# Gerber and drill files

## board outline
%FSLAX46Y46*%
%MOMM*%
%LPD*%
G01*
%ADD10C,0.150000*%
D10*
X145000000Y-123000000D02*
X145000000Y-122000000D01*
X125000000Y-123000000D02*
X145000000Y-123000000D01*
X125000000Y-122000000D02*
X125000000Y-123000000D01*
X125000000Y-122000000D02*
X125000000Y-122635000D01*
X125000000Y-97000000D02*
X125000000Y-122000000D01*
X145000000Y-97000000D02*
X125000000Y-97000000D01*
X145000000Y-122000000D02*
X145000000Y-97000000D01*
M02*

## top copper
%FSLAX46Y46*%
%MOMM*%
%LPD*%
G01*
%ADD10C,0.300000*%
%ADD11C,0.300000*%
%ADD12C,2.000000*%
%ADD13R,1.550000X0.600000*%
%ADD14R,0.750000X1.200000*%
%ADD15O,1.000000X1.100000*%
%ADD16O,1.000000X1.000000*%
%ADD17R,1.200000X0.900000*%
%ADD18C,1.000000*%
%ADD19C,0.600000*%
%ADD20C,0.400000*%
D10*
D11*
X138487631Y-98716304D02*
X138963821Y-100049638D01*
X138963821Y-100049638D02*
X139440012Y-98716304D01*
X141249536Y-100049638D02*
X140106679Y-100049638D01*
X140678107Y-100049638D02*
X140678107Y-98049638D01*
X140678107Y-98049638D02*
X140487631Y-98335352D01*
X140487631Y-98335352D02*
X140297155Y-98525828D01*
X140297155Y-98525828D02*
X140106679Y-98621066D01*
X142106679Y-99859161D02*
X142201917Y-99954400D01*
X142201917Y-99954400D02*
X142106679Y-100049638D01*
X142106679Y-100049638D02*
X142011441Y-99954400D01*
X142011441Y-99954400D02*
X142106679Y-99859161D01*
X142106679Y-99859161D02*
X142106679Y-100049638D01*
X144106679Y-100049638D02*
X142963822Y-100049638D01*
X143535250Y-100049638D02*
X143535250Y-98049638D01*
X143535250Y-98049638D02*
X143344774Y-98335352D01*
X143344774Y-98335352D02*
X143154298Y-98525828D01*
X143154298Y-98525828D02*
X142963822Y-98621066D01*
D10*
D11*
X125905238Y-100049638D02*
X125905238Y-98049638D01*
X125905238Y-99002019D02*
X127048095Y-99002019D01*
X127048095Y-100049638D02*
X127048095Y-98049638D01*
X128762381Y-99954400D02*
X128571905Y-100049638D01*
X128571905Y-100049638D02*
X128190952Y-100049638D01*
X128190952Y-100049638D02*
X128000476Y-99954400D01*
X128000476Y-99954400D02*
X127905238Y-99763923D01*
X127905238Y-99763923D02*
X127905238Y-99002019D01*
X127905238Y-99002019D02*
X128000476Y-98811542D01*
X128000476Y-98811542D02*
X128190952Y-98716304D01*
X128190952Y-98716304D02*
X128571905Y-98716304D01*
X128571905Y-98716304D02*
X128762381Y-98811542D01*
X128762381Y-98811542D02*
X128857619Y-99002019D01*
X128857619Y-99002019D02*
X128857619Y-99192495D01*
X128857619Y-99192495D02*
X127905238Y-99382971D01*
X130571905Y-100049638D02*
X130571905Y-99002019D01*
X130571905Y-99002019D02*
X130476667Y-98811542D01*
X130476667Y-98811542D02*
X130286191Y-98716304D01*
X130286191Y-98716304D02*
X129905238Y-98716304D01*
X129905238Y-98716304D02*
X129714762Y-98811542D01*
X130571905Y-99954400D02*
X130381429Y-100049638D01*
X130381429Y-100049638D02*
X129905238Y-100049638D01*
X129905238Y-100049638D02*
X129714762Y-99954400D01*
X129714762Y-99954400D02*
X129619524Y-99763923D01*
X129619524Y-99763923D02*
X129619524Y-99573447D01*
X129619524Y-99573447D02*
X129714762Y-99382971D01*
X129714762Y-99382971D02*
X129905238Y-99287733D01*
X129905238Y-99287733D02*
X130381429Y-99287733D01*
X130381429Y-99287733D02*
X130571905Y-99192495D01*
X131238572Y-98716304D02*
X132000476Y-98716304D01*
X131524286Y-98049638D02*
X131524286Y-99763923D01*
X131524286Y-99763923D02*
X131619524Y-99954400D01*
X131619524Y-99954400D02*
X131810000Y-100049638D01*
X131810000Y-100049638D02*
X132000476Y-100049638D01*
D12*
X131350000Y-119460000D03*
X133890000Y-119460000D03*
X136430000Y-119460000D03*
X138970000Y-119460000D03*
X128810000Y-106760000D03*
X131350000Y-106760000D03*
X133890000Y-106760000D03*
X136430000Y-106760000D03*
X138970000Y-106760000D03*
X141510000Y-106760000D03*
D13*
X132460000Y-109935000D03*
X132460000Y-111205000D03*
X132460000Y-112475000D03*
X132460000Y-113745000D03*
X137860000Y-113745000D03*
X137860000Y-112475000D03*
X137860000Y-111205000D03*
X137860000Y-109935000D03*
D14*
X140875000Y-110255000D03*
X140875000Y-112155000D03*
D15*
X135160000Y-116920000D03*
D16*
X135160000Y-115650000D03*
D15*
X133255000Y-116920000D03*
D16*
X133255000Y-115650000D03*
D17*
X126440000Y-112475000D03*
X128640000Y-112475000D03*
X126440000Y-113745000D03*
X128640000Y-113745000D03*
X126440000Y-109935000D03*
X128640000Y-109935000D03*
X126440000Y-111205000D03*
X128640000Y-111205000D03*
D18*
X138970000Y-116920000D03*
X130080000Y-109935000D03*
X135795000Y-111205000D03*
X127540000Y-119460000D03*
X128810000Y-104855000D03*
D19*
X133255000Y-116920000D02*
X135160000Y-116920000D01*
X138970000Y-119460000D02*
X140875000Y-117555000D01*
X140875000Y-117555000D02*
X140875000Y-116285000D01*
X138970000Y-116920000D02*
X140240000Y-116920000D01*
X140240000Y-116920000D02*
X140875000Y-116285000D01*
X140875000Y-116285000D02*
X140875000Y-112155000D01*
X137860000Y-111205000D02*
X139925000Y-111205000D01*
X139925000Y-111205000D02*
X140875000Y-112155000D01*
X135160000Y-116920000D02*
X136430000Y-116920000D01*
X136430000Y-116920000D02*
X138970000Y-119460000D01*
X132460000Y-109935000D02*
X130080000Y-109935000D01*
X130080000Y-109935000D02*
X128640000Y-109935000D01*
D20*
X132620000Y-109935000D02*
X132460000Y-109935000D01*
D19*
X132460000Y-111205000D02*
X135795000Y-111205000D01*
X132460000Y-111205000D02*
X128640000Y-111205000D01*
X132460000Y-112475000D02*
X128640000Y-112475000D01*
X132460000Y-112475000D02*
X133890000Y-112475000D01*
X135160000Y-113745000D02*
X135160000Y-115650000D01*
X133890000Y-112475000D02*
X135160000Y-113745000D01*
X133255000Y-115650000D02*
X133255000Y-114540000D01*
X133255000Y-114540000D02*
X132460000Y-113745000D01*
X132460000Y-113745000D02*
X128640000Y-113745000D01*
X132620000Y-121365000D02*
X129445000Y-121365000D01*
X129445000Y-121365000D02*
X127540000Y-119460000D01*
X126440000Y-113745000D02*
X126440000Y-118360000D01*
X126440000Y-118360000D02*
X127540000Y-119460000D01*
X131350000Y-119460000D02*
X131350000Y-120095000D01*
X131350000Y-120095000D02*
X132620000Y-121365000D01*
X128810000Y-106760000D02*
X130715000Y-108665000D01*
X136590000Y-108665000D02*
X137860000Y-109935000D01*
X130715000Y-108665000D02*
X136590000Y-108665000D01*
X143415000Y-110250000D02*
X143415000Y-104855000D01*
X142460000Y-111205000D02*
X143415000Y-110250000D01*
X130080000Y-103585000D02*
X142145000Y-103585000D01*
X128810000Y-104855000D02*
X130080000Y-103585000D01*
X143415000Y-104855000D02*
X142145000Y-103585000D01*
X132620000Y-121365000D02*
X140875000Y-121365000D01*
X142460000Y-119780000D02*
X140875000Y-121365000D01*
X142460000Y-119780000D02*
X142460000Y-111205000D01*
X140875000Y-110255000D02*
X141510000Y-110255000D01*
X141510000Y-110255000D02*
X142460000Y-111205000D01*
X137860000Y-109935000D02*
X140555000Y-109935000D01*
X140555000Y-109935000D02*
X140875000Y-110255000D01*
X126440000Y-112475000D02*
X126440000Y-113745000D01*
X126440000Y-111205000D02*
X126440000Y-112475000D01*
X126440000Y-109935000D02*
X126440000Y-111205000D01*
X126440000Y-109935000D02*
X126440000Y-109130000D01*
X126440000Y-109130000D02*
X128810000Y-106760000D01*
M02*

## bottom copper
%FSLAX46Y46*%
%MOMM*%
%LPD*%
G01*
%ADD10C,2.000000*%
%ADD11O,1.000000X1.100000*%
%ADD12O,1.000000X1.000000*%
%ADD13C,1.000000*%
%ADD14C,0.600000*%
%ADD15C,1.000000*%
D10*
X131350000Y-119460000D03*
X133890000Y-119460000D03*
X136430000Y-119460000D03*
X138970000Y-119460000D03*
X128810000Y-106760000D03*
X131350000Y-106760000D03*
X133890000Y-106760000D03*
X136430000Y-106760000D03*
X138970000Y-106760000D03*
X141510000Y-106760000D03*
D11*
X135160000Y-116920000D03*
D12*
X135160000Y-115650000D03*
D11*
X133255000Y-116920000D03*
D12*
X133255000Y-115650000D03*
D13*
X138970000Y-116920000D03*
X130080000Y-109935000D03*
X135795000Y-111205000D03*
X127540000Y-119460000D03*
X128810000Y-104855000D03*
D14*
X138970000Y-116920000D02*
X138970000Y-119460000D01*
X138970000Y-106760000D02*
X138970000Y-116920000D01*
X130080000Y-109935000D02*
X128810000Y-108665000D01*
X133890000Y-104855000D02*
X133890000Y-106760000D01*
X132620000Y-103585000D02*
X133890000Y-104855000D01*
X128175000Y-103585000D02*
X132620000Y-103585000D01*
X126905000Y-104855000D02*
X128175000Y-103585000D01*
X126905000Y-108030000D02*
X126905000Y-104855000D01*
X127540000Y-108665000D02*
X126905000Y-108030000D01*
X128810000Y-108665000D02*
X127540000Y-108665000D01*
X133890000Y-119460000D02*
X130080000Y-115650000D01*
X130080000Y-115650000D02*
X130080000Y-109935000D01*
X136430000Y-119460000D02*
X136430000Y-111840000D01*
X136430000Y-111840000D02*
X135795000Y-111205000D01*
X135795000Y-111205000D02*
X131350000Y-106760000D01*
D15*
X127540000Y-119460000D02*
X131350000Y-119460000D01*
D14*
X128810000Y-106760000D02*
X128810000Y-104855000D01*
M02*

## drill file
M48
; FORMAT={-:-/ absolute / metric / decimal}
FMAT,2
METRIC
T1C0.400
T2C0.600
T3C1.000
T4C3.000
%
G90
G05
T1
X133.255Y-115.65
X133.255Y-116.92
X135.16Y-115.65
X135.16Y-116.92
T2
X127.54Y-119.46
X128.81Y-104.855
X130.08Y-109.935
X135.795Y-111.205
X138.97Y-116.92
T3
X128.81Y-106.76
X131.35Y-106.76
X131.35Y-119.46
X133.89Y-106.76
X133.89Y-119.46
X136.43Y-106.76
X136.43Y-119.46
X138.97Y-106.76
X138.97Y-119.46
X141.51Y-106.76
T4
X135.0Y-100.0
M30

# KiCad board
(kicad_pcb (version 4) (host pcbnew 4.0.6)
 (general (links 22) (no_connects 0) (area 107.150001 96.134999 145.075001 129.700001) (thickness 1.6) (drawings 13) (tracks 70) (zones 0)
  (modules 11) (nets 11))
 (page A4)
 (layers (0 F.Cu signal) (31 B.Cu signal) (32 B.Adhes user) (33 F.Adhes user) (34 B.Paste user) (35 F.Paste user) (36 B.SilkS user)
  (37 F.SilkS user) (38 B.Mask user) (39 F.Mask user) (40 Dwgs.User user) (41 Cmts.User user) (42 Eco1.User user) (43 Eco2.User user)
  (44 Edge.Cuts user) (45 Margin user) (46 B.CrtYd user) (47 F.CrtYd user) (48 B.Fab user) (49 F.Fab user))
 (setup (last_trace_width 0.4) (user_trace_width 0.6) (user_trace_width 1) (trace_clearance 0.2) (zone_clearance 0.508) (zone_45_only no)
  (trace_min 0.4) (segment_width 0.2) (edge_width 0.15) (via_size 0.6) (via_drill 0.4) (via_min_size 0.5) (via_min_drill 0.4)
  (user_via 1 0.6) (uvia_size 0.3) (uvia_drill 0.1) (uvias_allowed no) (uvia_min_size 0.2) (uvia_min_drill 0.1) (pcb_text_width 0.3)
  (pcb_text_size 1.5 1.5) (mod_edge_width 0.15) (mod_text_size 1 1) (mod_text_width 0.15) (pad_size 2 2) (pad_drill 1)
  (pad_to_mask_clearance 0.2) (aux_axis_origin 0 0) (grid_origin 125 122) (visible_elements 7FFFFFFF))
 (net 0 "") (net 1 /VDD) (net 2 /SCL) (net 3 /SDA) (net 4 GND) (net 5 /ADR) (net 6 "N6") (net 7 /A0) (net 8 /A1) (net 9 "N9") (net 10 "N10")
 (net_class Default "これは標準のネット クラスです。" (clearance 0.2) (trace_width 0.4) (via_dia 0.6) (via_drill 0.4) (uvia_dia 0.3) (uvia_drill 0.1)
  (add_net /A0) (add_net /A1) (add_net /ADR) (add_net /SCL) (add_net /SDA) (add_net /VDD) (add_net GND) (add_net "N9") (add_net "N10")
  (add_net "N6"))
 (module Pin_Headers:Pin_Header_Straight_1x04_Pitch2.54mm (layer F.Cu) (at 131.35 119.46 90)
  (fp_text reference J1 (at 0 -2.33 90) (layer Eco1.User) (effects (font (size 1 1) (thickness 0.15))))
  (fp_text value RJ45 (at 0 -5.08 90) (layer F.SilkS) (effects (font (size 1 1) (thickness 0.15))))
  (pad 1 thru_hole circle (at 0 0 90) (size 2 2) (drill 1) (layers *.Cu *.Mask) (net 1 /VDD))
  (pad 2 thru_hole circle (at 0 2.54 90) (size 2 2) (drill 1) (layers *.Cu *.Mask) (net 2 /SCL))
  (pad 3 thru_hole circle (at 0 5.08 90) (size 2 2) (drill 1) (layers *.Cu *.Mask) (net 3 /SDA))
  (pad 4 thru_hole circle (at 0 7.62 90) (size 2 2) (drill 1) (layers *.Cu *.Mask) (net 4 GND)))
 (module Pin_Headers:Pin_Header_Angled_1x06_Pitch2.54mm (layer F.Cu) (at 128.81 106.76 90)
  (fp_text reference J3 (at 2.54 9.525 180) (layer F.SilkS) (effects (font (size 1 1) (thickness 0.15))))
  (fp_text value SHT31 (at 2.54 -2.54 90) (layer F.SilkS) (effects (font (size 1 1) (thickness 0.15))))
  (pad 1 thru_hole circle (at 0 0 90) (size 2 2) (drill 1) (layers *.Cu *.Mask) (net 1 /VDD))
  (pad 2 thru_hole circle (at 0 2.54 90) (size 2 2) (drill 1) (layers *.Cu *.Mask) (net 3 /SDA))
  (pad 3 thru_hole circle (at 0 5.08 90) (size 2 2) (drill 1) (layers *.Cu *.Mask) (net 2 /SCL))
  (pad 4 thru_hole circle (at 0 7.62 90) (size 2 2) (drill 1) (layers *.Cu *.Mask) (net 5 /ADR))
  (pad 5 thru_hole circle (at 0 10.16 90) (size 2 2) (drill 1) (layers *.Cu *.Mask) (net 4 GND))
  (pad 6 thru_hole circle (at 0 12.7 90) (size 2 2) (drill 1) (layers *.Cu *.Mask) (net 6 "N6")))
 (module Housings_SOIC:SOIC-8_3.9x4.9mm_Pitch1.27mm (layer F.Cu) (at 135.16 111.84)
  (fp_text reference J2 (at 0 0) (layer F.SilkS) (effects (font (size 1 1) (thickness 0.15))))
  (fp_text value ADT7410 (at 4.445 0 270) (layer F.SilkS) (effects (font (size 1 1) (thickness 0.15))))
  (pad 1 smd rect (at -2.7 -1.905) (size 1.55 0.6) (layers F.Cu F.Paste F.Mask) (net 2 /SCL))
  (pad 2 smd rect (at -2.7 -0.635) (size 1.55 0.6) (layers F.Cu F.Paste F.Mask) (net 3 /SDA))
  (pad 3 smd rect (at -2.7 0.635) (size 1.55 0.6) (layers F.Cu F.Paste F.Mask) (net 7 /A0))
  (pad 4 smd rect (at -2.7 1.905) (size 1.55 0.6) (layers F.Cu F.Paste F.Mask) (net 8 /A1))
  (pad 5 smd rect (at 2.7 1.905) (size 1.55 0.6) (layers F.Cu F.Paste F.Mask) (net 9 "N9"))
  (pad 6 smd rect (at 2.7 0.635) (size 1.55 0.6) (layers F.Cu F.Paste F.Mask) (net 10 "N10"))
  (pad 7 smd rect (at 2.7 -0.635) (size 1.55 0.6) (layers F.Cu F.Paste F.Mask) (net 4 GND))
  (pad 8 smd rect (at 2.7 -1.905) (size 1.55 0.6) (layers F.Cu F.Paste F.Mask) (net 1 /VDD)))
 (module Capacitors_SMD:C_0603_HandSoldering (layer F.Cu) (at 140.875 111.205 270)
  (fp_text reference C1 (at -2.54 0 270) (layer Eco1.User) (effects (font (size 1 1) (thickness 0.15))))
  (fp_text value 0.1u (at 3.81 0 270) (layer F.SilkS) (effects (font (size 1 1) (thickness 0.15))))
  (pad 1 smd rect (at -0.95 0 270) (size 1.2 0.75) (layers F.Cu F.Paste F.Mask) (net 1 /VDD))
  (pad 2 smd rect (at 0.95 0 270) (size 1.2 0.75) (layers F.Cu F.Paste F.Mask) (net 4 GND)))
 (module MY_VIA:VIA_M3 (layer F.Cu) (at 135 100)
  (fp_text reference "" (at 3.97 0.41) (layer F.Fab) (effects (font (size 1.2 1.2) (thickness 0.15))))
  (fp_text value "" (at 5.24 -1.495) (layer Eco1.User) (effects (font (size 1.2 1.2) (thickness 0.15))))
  (pad "" np_thru_hole oval (at 0 0) (size 3 3) (drill 3) (layers *.Cu *.Mask)))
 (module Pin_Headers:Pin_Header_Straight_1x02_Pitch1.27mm (layer F.Cu) (at 135.16 116.92 180)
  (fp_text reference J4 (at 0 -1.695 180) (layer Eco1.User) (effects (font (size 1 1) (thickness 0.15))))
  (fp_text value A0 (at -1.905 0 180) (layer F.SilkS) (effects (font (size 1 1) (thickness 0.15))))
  (pad 1 thru_hole oval (at 0 0 180) (size 1 1.1) (drill 0.4) (layers *.Cu *.Mask) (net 4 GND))
  (pad 2 thru_hole oval (at 0 1.27 180) (size 1 1) (drill 0.4) (layers *.Cu *.Mask) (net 7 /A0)))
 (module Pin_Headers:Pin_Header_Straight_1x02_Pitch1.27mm (layer F.Cu) (at 133.255 116.92 180)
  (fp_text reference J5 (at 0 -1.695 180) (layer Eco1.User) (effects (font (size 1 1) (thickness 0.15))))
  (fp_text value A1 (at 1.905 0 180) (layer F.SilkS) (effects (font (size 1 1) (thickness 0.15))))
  (pad 1 thru_hole oval (at 0 0 180) (size 1 1.1) (drill 0.4) (layers *.Cu *.Mask) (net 4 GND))
  (pad 2 thru_hole oval (at 0 1.27 180) (size 1 1) (drill 0.4) (layers *.Cu *.Mask) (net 8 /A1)))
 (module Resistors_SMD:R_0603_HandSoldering (layer F.Cu) (at 127.54 112.475)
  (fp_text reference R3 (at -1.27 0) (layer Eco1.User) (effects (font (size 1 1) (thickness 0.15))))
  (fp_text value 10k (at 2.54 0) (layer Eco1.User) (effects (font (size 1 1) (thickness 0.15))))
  (pad 1 smd rect (at -1.1 0) (size 1.2 0.9) (layers F.Cu F.Paste F.Mask) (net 1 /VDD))
  (pad 2 smd rect (at 1.1 0) (size 1.2 0.9) (layers F.Cu F.Paste F.Mask) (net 7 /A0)))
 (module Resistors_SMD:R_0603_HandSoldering (layer F.Cu) (at 127.54 113.745)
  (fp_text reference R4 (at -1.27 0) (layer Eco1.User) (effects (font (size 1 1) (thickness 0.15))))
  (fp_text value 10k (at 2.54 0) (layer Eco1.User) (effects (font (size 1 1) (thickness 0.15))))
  (pad 1 smd rect (at -1.1 0) (size 1.2 0.9) (layers F.Cu F.Paste F.Mask) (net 1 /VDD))
  (pad 2 smd rect (at 1.1 0) (size 1.2 0.9) (layers F.Cu F.Paste F.Mask) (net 8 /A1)))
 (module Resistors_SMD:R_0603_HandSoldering (layer F.Cu) (at 127.54 109.935)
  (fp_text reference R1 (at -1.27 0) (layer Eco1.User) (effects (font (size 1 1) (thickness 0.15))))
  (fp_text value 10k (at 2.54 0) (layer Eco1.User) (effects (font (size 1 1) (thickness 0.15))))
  (pad 1 smd rect (at -1.1 0) (size 1.2 0.9) (layers F.Cu F.Paste F.Mask) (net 1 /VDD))
  (pad 2 smd rect (at 1.1 0) (size 1.2 0.9) (layers F.Cu F.Paste F.Mask) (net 2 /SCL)))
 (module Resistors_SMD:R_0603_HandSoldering (layer F.Cu) (at 127.54 111.205)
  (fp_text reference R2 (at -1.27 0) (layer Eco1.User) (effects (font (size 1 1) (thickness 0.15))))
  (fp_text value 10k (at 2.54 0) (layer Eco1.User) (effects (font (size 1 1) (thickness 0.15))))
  (pad 1 smd rect (at -1.1 0) (size 1.2 0.9) (layers F.Cu F.Paste F.Mask) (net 1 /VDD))
  (pad 2 smd rect (at 1.1 0) (size 1.2 0.9) (layers F.Cu F.Paste F.Mask) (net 3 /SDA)))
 (gr_line (start 145 123) (end 145 122) (angle 90) (layer Edge.Cuts) (width 0.15))
 (gr_line (start 125 123) (end 145 123) (angle 90) (layer Edge.Cuts) (width 0.15))
 (gr_line (start 125 122) (end 125 123) (angle 90) (layer Edge.Cuts) (width 0.15))
 (gr_line (start 125 122) (end 125 122.635) (angle 90) (layer Edge.Cuts) (width 0.15))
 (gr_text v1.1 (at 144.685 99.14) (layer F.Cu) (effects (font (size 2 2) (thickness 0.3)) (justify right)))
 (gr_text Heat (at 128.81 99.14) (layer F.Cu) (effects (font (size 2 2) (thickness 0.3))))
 (gr_line (start 125 97) (end 125 122) (angle 90) (layer Edge.Cuts) (width 0.15))
 (gr_line (start 145 97) (end 125 97) (angle 90) (layer Edge.Cuts) (width 0.15))
 (gr_line (start 145 122) (end 145 97) (angle 90) (layer Edge.Cuts) (width 0.15))
 (segment (start 133.255 116.92) (end 135.16 116.92) (width 0.6) (layer F.Cu) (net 4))
 (segment (start 138.97 116.92) (end 138.97 119.46) (width 0.6) (layer B.Cu) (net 4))
 (segment (start 138.97 119.46) (end 140.875 117.555) (width 0.6) (layer F.Cu) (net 4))
 (segment (start 140.875 117.555) (end 140.875 116.285) (width 0.6) (layer F.Cu) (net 4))
 (segment (start 138.97 116.92) (end 140.24 116.92) (width 0.6) (layer F.Cu) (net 4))
 (segment (start 140.24 116.92) (end 140.875 116.285) (width 0.6) (layer F.Cu) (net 4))
 (via (at 138.97 116.92) (size 1) (drill 0.6) (layers F.Cu B.Cu) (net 4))
 (segment (start 140.875 116.285) (end 140.875 112.155) (width 0.6) (layer F.Cu) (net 4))
 (segment (start 137.86 111.205) (end 139.925 111.205) (width 0.6) (layer F.Cu) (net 4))
 (segment (start 139.925 111.205) (end 140.875 112.155) (width 0.6) (layer F.Cu) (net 4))
 (segment (start 138.97 106.76) (end 138.97 116.92) (width 0.6) (layer B.Cu) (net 4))
 (segment (start 135.16 116.92) (end 136.43 116.92) (width 0.6) (layer F.Cu) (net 4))
 (segment (start 136.43 116.92) (end 138.97 119.46) (width 0.6) (layer F.Cu) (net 4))
 (segment (start 130.08 109.935) (end 128.81 108.665) (width 0.6) (layer B.Cu) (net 2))
 (segment (start 133.89 104.855) (end 133.89 106.76) (width 0.6) (layer B.Cu) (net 2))
 (segment (start 132.62 103.585) (end 133.89 104.855) (width 0.6) (layer B.Cu) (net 2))
 (segment (start 128.175 103.585) (end 132.62 103.585) (width 0.6) (layer B.Cu) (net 2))
 (segment (start 126.905 104.855) (end 128.175 103.585) (width 0.6) (layer B.Cu) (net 2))
 (segment (start 126.905 108.03) (end 126.905 104.855) (width 0.6) (layer B.Cu) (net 2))
 (segment (start 127.54 108.665) (end 126.905 108.03) (width 0.6) (layer B.Cu) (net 2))
 (segment (start 128.81 108.665) (end 127.54 108.665) (width 0.6) (layer B.Cu) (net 2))
 (segment (start 133.89 119.46) (end 130.08 115.65) (width 0.6) (layer B.Cu) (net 2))
 (via (at 130.08 109.935) (size 1) (drill 0.6) (layers F.Cu B.Cu) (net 2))
 (segment (start 130.08 115.65) (end 130.08 109.935) (width 0.6) (layer B.Cu) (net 2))
 (segment (start 132.46 109.935) (end 130.08 109.935) (width 0.6) (layer F.Cu) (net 2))
 (segment (start 130.08 109.935) (end 128.64 109.935) (width 0.6) (layer F.Cu) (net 2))
 (segment (start 132.62 109.935) (end 132.46 109.935) (width 0.4) (layer F.Cu) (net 2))
 (segment (start 132.46 111.205) (end 135.795 111.205) (width 0.6) (layer F.Cu) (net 3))
 (via (at 135.795 111.205) (size 1) (drill 0.6) (layers F.Cu B.Cu) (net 3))
 (segment (start 136.43 119.46) (end 136.43 111.84) (width 0.6) (layer B.Cu) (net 3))
 (segment (start 136.43 111.84) (end 135.795 111.205) (width 0.6) (layer B.Cu) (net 3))
 (segment (start 135.795 111.205) (end 131.35 106.76) (width 0.6) (layer B.Cu) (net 3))
 (segment (start 132.46 111.205) (end 128.64 111.205) (width 0.6) (layer F.Cu) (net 3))
 (segment (start 132.46 112.475) (end 128.64 112.475) (width 0.6) (layer F.Cu) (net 7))
 (segment (start 132.46 112.475) (end 133.89 112.475) (width 0.6) (layer F.Cu) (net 7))
 (segment (start 135.16 113.745) (end 135.16 115.65) (width 0.6) (layer F.Cu) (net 7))
 (segment (start 133.89 112.475) (end 135.16 113.745) (width 0.6) (layer F.Cu) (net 7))
 (segment (start 133.255 115.65) (end 133.255 114.54) (width 0.6) (layer F.Cu) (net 8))
 (segment (start 133.255 114.54) (end 132.46 113.745) (width 0.6) (layer F.Cu) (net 8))
 (segment (start 132.46 113.745) (end 128.64 113.745) (width 0.6) (layer F.Cu) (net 8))
 (segment (start 132.62 121.365) (end 129.445 121.365) (width 0.6) (layer F.Cu) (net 1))
 (segment (start 129.445 121.365) (end 127.54 119.46) (width 0.6) (layer F.Cu) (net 1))
 (segment (start 126.44 113.745) (end 126.44 118.36) (width 0.6) (layer F.Cu) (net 1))
 (segment (start 126.44 118.36) (end 127.54 119.46) (width 0.6) (layer F.Cu) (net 1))
 (via (at 127.54 119.46) (size 1) (drill 0.6) (layers F.Cu B.Cu) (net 1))
 (segment (start 127.54 119.46) (end 131.35 119.46) (width 1) (layer B.Cu) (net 1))
 (segment (start 131.35 119.46) (end 131.35 120.095) (width 0.6) (layer F.Cu) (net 1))
 (segment (start 131.35 120.095) (end 132.62 121.365) (width 0.6) (layer F.Cu) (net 1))
 (segment (start 128.81 106.76) (end 130.715 108.665) (width 0.6) (layer F.Cu) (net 1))
 (segment (start 136.59 108.665) (end 137.86 109.935) (width 0.6) (layer F.Cu) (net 1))
 (segment (start 130.715 108.665) (end 136.59 108.665) (width 0.6) (layer F.Cu) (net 1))
 (segment (start 128.81 106.76) (end 128.81 104.855) (width 0.6) (layer B.Cu) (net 1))
 (via (at 128.81 104.855) (size 1) (drill 0.6) (layers F.Cu B.Cu) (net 1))
 (segment (start 143.415 110.25) (end 143.415 104.855) (width 0.6) (layer F.Cu) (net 1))
 (segment (start 142.46 111.205) (end 143.415 110.25) (width 0.6) (layer F.Cu) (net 1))
 (segment (start 130.08 103.585) (end 142.145 103.585) (width 0.6) (layer F.Cu) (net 1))
 (segment (start 128.81 104.855) (end 130.08 103.585) (width 0.6) (layer F.Cu) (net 1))
 (segment (start 143.415 104.855) (end 142.145 103.585) (width 0.6) (layer F.Cu) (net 1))
 (segment (start 132.62 121.365) (end 140.875 121.365) (width 0.6) (layer F.Cu) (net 1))
 (segment (start 142.46 119.78) (end 140.875 121.365) (width 0.6) (layer F.Cu) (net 1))
 (segment (start 142.46 119.78) (end 142.46 111.205) (width 0.6) (layer F.Cu) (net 1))
 (segment (start 140.875 110.255) (end 141.51 110.255) (width 0.6) (layer F.Cu) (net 1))
 (segment (start 141.51 110.255) (end 142.46 111.205) (width 0.6) (layer F.Cu) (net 1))
 (segment (start 137.86 109.935) (end 140.555 109.935) (width 0.6) (layer F.Cu) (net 1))
 (segment (start 140.555 109.935) (end 140.875 110.255) (width 0.6) (layer F.Cu) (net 1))
 (segment (start 126.44 112.475) (end 126.44 113.745) (width 0.6) (layer F.Cu) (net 1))
 (segment (start 126.44 111.205) (end 126.44 112.475) (width 0.6) (layer F.Cu) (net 1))
 (segment (start 126.44 109.935) (end 126.44 111.205) (width 0.6) (layer F.Cu) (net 1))
 (segment (start 126.44 109.935) (end 126.44 109.13) (width 0.6) (layer F.Cu) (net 1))
 (segment (start 126.44 109.13) (end 128.81 106.76) (width 0.6) (layer F.Cu) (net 1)))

